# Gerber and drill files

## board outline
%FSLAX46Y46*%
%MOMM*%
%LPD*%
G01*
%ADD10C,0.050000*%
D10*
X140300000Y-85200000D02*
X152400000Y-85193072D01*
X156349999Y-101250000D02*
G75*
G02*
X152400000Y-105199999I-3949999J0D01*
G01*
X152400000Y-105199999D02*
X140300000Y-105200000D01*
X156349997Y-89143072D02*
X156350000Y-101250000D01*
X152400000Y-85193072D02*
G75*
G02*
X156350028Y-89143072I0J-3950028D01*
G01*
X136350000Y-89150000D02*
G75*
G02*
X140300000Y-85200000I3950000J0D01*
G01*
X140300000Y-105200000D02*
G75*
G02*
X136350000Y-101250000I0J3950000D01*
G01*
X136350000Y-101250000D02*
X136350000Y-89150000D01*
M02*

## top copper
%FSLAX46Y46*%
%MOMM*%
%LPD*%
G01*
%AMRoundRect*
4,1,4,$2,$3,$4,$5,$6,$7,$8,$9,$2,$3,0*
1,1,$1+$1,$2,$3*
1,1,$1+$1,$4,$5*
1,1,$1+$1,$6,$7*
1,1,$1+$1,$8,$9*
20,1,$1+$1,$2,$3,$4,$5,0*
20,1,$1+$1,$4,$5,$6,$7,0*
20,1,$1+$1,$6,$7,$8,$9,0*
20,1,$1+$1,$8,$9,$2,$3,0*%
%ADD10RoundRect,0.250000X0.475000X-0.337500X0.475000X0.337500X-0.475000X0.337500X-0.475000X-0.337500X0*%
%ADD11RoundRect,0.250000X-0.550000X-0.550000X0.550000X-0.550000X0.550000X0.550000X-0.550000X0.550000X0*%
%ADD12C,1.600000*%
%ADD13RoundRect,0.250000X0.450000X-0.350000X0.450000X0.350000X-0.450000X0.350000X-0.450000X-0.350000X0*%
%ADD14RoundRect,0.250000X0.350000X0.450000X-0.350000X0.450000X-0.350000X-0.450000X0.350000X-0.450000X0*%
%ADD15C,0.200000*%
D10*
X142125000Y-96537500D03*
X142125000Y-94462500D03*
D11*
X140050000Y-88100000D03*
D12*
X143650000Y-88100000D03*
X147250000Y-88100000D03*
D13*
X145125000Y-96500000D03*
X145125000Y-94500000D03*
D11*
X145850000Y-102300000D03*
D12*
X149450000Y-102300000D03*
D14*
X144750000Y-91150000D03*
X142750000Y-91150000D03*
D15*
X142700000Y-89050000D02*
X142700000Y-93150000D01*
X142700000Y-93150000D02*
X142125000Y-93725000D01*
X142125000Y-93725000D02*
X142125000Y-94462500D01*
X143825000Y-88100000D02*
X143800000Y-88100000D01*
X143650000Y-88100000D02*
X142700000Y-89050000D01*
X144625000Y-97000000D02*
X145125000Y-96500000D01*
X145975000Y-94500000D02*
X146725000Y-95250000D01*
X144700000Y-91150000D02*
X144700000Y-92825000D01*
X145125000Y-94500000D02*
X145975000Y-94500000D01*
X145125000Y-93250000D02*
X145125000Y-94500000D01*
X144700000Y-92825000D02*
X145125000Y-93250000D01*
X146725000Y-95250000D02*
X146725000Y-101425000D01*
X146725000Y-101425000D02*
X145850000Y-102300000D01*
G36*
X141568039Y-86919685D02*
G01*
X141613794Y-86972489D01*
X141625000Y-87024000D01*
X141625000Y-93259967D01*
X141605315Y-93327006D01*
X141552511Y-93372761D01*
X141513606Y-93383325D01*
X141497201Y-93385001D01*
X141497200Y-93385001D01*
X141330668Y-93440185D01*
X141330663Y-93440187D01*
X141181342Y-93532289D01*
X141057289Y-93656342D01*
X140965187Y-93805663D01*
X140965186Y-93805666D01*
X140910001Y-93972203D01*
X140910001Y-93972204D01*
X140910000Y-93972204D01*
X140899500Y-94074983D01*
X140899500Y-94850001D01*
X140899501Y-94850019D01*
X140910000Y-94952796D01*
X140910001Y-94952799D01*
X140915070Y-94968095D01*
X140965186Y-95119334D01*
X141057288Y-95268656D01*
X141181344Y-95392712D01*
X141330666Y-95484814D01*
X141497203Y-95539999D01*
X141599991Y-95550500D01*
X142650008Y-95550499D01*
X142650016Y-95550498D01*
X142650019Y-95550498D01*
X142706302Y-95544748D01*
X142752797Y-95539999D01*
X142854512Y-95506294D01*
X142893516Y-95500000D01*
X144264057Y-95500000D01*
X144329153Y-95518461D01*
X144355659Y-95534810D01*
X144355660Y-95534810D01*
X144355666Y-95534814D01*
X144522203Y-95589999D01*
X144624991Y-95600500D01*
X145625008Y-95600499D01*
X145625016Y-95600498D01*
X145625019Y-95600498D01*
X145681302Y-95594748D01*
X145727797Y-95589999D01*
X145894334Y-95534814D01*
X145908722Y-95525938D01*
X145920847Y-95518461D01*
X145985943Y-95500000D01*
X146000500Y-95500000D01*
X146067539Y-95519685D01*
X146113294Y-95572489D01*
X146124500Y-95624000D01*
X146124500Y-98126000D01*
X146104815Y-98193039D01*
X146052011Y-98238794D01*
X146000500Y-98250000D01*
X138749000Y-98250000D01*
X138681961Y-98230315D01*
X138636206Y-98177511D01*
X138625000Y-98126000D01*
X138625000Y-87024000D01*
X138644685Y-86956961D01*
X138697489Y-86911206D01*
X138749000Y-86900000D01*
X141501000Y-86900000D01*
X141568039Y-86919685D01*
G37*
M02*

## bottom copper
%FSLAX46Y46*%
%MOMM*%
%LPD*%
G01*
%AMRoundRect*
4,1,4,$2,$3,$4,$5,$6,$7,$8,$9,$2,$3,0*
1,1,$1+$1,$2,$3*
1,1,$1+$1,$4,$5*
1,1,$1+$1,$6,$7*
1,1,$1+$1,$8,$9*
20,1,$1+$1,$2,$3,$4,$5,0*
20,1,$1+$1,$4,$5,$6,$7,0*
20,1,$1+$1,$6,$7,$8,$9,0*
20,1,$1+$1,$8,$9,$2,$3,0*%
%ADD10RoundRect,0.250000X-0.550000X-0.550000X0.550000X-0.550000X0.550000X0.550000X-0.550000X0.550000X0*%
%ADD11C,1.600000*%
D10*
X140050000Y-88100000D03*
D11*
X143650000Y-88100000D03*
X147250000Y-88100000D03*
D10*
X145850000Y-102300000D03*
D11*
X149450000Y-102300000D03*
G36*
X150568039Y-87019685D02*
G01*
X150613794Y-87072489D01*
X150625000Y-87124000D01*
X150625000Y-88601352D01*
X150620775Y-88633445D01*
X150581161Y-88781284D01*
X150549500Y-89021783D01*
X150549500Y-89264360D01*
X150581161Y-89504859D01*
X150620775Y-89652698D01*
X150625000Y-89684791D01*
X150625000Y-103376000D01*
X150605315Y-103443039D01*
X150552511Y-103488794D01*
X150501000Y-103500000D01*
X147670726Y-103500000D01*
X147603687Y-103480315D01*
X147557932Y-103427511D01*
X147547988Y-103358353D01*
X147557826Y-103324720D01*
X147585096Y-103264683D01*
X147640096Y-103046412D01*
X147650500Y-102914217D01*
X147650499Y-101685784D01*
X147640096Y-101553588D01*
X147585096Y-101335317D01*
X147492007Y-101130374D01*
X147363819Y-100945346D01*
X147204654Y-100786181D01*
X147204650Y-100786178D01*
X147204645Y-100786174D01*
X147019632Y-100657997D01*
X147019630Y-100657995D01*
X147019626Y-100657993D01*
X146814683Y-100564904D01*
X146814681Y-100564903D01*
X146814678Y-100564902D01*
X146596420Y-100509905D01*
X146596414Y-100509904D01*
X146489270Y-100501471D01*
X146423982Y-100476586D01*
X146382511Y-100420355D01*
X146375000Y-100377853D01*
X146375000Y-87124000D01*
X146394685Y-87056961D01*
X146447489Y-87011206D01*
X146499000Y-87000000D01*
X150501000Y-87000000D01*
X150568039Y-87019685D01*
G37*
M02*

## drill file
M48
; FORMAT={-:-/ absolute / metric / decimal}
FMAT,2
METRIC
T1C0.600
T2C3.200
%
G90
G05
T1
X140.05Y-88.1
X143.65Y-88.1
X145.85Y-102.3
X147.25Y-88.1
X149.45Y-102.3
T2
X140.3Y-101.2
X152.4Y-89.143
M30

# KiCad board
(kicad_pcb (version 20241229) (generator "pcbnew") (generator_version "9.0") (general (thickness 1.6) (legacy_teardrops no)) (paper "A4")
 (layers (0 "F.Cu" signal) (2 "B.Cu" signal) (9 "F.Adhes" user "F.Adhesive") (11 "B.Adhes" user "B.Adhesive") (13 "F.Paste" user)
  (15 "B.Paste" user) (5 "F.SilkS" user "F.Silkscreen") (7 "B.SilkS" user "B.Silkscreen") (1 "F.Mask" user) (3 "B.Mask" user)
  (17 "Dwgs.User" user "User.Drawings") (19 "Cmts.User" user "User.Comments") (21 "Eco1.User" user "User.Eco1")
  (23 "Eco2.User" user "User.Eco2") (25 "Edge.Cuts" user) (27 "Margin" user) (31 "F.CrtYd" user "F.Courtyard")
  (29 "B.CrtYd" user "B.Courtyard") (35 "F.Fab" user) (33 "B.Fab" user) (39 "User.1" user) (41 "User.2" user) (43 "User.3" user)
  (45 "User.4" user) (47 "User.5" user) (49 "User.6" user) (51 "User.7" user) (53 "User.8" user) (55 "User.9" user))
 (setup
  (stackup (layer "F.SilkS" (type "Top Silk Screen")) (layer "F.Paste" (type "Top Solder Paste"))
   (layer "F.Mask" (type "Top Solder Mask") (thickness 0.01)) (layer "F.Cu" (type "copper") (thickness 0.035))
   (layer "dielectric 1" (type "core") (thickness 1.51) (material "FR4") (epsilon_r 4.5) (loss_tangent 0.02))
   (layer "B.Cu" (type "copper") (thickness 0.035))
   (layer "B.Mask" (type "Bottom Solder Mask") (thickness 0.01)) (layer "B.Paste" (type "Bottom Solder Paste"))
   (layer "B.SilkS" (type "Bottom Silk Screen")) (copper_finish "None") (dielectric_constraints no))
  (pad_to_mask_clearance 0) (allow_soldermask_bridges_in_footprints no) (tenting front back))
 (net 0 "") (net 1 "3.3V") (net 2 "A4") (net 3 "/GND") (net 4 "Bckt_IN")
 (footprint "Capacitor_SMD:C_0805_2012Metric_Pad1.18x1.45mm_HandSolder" (layer "F.Cu") (at 142.125 95.5 90)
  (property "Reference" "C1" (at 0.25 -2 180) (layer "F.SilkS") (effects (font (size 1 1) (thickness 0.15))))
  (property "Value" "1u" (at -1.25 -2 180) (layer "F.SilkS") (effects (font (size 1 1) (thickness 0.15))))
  (pad "1" smd roundrect (at -1.0375 0 90) (size 1.175 1.45) (layers "F.Cu" "F.Mask" "F.Paste") (roundrect_rratio 0.212766) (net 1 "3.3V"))
  (pad "2" smd roundrect (at 1.0375 0 90) (size 1.175 1.45) (layers "F.Cu" "F.Mask" "F.Paste") (roundrect_rratio 0.212766) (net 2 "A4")))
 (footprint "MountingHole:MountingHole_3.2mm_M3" (layer "F.Cu") (at 152.4 89.143072)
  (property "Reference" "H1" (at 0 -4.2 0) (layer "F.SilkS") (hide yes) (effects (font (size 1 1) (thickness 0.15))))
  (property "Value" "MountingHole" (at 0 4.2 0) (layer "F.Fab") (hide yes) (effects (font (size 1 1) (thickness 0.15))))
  (pad "" np_thru_hole circle (at 0 0) (size 3.2 3.2) (drill 3.2) (layers "*.Cu" "*.Mask")))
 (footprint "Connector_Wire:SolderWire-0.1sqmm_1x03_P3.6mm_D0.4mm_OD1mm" (layer "F.Cu") (at 140.05 88.1)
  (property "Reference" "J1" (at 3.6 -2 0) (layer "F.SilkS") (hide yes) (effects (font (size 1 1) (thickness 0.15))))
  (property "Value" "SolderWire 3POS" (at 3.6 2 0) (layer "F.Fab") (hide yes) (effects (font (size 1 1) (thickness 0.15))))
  (pad "1" thru_hole roundrect (at 0 0) (size 1.6 1.6) (drill 0.6) (layers "*.Cu" "*.Mask") (remove_unused_layers no)
   (roundrect_rratio 0.15625) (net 1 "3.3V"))
  (pad "2" thru_hole circle (at 3.6 0) (size 1.6 1.6) (drill 0.6) (layers "*.Cu" "*.Mask") (remove_unused_layers no) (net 2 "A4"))
  (pad "3" thru_hole circle (at 7.2 0) (size 1.6 1.6) (drill 0.6) (layers "*.Cu" "*.Mask") (remove_unused_layers no) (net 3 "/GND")))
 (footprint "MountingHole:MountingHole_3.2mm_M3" (layer "F.Cu") (at 140.3 101.2)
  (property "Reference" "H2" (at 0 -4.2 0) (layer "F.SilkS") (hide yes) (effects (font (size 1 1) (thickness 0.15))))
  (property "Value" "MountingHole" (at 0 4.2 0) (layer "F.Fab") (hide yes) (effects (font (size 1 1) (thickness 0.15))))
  (pad "" np_thru_hole circle (at 0 0) (size 3.2 3.2) (drill 3.2) (layers "*.Cu" "*.Mask")))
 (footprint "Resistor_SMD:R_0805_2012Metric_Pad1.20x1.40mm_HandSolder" (layer "F.Cu") (at 145.125 95.5 90)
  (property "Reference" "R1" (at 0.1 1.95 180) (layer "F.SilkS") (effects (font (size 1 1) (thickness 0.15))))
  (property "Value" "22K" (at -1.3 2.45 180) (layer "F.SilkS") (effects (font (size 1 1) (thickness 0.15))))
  (pad "1" smd roundrect (at -1 0 90) (size 1.2 1.4) (layers "F.Cu" "F.Mask" "F.Paste") (roundrect_rratio 0.208333) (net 1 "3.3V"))
  (pad "2" smd roundrect (at 1 0 90) (size 1.2 1.4) (layers "F.Cu" "F.Mask" "F.Paste") (roundrect_rratio 0.208333) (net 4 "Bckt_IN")))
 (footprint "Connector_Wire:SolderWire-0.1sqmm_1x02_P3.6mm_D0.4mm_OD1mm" (layer "F.Cu") (at 145.85 102.3)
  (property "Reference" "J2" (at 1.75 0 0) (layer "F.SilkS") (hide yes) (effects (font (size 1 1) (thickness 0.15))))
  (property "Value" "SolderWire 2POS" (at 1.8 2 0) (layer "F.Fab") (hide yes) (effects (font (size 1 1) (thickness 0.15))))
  (pad "1" thru_hole roundrect (at 0 0) (size 1.6 1.6) (drill 0.6) (layers "*.Cu" "*.Mask") (remove_unused_layers no)
   (roundrect_rratio 0.15625) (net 4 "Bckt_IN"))
  (pad "2" thru_hole circle (at 3.6 0) (size 1.6 1.6) (drill 0.6) (layers "*.Cu" "*.Mask") (remove_unused_layers no) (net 3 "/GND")))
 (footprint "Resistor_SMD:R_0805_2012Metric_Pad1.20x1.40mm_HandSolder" (layer "F.Cu") (at 143.75 91.15 180)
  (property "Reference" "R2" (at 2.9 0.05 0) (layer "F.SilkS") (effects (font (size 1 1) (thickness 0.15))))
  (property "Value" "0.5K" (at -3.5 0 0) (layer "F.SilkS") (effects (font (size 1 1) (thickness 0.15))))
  (pad "1" smd roundrect (at -1 0 180) (size 1.2 1.4) (layers "F.Cu" "F.Mask" "F.Paste") (roundrect_rratio 0.208333) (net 4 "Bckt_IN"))
  (pad "2" smd roundrect (at 1 0 180) (size 1.2 1.4) (layers "F.Cu" "F.Mask" "F.Paste") (roundrect_rratio 0.208333) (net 2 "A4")))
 (gr_line (start 140.3 85.2) (end 152.4 85.193072) (stroke (width 0.05) (type default)) (layer "Edge.Cuts"))
 (gr_arc (start 156.349999 101.25) (mid 155.193071 104.043071) (end 152.4 105.199999) (stroke (width 0.05) (type default))
  (layer "Edge.Cuts"))
 (gr_line (start 152.4 105.199999) (end 140.3 105.2) (stroke (width 0.05) (type default)) (layer "Edge.Cuts"))
 (gr_line (start 156.349997 89.143072) (end 156.35 101.25) (stroke (width 0.05) (type default)) (layer "Edge.Cuts"))
 (gr_arc (start 152.4 85.193072) (mid 155.193072 86.35) (end 156.35 89.143072) (stroke (width 0.05) (type default)) (layer "Edge.Cuts"))
 (gr_arc (start 136.35 89.15) (mid 137.506928 86.356928) (end 140.3 85.2) (stroke (width 0.05) (type default)) (layer "Edge.Cuts"))
 (gr_arc (start 140.3 105.2) (mid 137.506928 104.043072) (end 136.35 101.25) (stroke (width 0.05) (type default)) (layer "Edge.Cuts"))
 (gr_line (start 136.35 101.25) (end 136.35 89.15) (stroke (width 0.05) (type default)) (layer "Edge.Cuts"))
 (segment (start 142.7 89.05) (end 142.7 93.15) (width 0.2) (layer "F.Cu") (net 2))
 (segment (start 142.7 93.15) (end 142.125 93.725) (width 0.2) (layer "F.Cu") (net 2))
 (segment (start 142.125 93.725) (end 142.125 94.4625) (width 0.2) (layer "F.Cu") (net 2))
 (segment (start 143.825 88.1) (end 143.8 88.1) (width 0.2) (layer "F.Cu") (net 2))
 (segment (start 143.65 88.1) (end 142.7 89.05) (width 0.2) (layer "F.Cu") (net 2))
 (segment (start 144.625 97) (end 145.125 96.5) (width 0.2) (layer "F.Cu") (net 1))
 (segment (start 145.975 94.5) (end 146.725 95.25) (width 0.2) (layer "F.Cu") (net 4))
 (segment (start 144.7 91.15) (end 144.7 92.825) (width 0.2) (layer "F.Cu") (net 4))
 (segment (start 145.125 94.5) (end 145.975 94.5) (width 0.2) (layer "F.Cu") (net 4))
 (segment (start 145.125 93.25) (end 145.125 94.5) (width 0.2) (layer "F.Cu") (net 4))
 (segment (start 144.7 92.825) (end 145.125 93.25) (width 0.2) (layer "F.Cu") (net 4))
 (segment (start 146.725 95.25) (end 146.725 101.425) (width 0.2) (layer "F.Cu") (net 4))
 (segment (start 146.725 101.425) (end 145.85 102.3) (width 0.2) (layer "F.Cu") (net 4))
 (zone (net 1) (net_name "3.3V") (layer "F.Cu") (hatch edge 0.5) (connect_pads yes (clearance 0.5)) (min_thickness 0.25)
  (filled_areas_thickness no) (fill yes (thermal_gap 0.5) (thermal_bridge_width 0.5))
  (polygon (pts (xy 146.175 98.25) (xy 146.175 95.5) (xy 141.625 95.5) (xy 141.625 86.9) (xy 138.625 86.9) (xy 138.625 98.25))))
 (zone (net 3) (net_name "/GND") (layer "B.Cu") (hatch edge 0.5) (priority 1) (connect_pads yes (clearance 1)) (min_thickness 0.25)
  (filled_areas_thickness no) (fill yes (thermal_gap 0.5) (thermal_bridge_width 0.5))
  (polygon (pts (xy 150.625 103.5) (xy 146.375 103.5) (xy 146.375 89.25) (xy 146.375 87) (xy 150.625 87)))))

